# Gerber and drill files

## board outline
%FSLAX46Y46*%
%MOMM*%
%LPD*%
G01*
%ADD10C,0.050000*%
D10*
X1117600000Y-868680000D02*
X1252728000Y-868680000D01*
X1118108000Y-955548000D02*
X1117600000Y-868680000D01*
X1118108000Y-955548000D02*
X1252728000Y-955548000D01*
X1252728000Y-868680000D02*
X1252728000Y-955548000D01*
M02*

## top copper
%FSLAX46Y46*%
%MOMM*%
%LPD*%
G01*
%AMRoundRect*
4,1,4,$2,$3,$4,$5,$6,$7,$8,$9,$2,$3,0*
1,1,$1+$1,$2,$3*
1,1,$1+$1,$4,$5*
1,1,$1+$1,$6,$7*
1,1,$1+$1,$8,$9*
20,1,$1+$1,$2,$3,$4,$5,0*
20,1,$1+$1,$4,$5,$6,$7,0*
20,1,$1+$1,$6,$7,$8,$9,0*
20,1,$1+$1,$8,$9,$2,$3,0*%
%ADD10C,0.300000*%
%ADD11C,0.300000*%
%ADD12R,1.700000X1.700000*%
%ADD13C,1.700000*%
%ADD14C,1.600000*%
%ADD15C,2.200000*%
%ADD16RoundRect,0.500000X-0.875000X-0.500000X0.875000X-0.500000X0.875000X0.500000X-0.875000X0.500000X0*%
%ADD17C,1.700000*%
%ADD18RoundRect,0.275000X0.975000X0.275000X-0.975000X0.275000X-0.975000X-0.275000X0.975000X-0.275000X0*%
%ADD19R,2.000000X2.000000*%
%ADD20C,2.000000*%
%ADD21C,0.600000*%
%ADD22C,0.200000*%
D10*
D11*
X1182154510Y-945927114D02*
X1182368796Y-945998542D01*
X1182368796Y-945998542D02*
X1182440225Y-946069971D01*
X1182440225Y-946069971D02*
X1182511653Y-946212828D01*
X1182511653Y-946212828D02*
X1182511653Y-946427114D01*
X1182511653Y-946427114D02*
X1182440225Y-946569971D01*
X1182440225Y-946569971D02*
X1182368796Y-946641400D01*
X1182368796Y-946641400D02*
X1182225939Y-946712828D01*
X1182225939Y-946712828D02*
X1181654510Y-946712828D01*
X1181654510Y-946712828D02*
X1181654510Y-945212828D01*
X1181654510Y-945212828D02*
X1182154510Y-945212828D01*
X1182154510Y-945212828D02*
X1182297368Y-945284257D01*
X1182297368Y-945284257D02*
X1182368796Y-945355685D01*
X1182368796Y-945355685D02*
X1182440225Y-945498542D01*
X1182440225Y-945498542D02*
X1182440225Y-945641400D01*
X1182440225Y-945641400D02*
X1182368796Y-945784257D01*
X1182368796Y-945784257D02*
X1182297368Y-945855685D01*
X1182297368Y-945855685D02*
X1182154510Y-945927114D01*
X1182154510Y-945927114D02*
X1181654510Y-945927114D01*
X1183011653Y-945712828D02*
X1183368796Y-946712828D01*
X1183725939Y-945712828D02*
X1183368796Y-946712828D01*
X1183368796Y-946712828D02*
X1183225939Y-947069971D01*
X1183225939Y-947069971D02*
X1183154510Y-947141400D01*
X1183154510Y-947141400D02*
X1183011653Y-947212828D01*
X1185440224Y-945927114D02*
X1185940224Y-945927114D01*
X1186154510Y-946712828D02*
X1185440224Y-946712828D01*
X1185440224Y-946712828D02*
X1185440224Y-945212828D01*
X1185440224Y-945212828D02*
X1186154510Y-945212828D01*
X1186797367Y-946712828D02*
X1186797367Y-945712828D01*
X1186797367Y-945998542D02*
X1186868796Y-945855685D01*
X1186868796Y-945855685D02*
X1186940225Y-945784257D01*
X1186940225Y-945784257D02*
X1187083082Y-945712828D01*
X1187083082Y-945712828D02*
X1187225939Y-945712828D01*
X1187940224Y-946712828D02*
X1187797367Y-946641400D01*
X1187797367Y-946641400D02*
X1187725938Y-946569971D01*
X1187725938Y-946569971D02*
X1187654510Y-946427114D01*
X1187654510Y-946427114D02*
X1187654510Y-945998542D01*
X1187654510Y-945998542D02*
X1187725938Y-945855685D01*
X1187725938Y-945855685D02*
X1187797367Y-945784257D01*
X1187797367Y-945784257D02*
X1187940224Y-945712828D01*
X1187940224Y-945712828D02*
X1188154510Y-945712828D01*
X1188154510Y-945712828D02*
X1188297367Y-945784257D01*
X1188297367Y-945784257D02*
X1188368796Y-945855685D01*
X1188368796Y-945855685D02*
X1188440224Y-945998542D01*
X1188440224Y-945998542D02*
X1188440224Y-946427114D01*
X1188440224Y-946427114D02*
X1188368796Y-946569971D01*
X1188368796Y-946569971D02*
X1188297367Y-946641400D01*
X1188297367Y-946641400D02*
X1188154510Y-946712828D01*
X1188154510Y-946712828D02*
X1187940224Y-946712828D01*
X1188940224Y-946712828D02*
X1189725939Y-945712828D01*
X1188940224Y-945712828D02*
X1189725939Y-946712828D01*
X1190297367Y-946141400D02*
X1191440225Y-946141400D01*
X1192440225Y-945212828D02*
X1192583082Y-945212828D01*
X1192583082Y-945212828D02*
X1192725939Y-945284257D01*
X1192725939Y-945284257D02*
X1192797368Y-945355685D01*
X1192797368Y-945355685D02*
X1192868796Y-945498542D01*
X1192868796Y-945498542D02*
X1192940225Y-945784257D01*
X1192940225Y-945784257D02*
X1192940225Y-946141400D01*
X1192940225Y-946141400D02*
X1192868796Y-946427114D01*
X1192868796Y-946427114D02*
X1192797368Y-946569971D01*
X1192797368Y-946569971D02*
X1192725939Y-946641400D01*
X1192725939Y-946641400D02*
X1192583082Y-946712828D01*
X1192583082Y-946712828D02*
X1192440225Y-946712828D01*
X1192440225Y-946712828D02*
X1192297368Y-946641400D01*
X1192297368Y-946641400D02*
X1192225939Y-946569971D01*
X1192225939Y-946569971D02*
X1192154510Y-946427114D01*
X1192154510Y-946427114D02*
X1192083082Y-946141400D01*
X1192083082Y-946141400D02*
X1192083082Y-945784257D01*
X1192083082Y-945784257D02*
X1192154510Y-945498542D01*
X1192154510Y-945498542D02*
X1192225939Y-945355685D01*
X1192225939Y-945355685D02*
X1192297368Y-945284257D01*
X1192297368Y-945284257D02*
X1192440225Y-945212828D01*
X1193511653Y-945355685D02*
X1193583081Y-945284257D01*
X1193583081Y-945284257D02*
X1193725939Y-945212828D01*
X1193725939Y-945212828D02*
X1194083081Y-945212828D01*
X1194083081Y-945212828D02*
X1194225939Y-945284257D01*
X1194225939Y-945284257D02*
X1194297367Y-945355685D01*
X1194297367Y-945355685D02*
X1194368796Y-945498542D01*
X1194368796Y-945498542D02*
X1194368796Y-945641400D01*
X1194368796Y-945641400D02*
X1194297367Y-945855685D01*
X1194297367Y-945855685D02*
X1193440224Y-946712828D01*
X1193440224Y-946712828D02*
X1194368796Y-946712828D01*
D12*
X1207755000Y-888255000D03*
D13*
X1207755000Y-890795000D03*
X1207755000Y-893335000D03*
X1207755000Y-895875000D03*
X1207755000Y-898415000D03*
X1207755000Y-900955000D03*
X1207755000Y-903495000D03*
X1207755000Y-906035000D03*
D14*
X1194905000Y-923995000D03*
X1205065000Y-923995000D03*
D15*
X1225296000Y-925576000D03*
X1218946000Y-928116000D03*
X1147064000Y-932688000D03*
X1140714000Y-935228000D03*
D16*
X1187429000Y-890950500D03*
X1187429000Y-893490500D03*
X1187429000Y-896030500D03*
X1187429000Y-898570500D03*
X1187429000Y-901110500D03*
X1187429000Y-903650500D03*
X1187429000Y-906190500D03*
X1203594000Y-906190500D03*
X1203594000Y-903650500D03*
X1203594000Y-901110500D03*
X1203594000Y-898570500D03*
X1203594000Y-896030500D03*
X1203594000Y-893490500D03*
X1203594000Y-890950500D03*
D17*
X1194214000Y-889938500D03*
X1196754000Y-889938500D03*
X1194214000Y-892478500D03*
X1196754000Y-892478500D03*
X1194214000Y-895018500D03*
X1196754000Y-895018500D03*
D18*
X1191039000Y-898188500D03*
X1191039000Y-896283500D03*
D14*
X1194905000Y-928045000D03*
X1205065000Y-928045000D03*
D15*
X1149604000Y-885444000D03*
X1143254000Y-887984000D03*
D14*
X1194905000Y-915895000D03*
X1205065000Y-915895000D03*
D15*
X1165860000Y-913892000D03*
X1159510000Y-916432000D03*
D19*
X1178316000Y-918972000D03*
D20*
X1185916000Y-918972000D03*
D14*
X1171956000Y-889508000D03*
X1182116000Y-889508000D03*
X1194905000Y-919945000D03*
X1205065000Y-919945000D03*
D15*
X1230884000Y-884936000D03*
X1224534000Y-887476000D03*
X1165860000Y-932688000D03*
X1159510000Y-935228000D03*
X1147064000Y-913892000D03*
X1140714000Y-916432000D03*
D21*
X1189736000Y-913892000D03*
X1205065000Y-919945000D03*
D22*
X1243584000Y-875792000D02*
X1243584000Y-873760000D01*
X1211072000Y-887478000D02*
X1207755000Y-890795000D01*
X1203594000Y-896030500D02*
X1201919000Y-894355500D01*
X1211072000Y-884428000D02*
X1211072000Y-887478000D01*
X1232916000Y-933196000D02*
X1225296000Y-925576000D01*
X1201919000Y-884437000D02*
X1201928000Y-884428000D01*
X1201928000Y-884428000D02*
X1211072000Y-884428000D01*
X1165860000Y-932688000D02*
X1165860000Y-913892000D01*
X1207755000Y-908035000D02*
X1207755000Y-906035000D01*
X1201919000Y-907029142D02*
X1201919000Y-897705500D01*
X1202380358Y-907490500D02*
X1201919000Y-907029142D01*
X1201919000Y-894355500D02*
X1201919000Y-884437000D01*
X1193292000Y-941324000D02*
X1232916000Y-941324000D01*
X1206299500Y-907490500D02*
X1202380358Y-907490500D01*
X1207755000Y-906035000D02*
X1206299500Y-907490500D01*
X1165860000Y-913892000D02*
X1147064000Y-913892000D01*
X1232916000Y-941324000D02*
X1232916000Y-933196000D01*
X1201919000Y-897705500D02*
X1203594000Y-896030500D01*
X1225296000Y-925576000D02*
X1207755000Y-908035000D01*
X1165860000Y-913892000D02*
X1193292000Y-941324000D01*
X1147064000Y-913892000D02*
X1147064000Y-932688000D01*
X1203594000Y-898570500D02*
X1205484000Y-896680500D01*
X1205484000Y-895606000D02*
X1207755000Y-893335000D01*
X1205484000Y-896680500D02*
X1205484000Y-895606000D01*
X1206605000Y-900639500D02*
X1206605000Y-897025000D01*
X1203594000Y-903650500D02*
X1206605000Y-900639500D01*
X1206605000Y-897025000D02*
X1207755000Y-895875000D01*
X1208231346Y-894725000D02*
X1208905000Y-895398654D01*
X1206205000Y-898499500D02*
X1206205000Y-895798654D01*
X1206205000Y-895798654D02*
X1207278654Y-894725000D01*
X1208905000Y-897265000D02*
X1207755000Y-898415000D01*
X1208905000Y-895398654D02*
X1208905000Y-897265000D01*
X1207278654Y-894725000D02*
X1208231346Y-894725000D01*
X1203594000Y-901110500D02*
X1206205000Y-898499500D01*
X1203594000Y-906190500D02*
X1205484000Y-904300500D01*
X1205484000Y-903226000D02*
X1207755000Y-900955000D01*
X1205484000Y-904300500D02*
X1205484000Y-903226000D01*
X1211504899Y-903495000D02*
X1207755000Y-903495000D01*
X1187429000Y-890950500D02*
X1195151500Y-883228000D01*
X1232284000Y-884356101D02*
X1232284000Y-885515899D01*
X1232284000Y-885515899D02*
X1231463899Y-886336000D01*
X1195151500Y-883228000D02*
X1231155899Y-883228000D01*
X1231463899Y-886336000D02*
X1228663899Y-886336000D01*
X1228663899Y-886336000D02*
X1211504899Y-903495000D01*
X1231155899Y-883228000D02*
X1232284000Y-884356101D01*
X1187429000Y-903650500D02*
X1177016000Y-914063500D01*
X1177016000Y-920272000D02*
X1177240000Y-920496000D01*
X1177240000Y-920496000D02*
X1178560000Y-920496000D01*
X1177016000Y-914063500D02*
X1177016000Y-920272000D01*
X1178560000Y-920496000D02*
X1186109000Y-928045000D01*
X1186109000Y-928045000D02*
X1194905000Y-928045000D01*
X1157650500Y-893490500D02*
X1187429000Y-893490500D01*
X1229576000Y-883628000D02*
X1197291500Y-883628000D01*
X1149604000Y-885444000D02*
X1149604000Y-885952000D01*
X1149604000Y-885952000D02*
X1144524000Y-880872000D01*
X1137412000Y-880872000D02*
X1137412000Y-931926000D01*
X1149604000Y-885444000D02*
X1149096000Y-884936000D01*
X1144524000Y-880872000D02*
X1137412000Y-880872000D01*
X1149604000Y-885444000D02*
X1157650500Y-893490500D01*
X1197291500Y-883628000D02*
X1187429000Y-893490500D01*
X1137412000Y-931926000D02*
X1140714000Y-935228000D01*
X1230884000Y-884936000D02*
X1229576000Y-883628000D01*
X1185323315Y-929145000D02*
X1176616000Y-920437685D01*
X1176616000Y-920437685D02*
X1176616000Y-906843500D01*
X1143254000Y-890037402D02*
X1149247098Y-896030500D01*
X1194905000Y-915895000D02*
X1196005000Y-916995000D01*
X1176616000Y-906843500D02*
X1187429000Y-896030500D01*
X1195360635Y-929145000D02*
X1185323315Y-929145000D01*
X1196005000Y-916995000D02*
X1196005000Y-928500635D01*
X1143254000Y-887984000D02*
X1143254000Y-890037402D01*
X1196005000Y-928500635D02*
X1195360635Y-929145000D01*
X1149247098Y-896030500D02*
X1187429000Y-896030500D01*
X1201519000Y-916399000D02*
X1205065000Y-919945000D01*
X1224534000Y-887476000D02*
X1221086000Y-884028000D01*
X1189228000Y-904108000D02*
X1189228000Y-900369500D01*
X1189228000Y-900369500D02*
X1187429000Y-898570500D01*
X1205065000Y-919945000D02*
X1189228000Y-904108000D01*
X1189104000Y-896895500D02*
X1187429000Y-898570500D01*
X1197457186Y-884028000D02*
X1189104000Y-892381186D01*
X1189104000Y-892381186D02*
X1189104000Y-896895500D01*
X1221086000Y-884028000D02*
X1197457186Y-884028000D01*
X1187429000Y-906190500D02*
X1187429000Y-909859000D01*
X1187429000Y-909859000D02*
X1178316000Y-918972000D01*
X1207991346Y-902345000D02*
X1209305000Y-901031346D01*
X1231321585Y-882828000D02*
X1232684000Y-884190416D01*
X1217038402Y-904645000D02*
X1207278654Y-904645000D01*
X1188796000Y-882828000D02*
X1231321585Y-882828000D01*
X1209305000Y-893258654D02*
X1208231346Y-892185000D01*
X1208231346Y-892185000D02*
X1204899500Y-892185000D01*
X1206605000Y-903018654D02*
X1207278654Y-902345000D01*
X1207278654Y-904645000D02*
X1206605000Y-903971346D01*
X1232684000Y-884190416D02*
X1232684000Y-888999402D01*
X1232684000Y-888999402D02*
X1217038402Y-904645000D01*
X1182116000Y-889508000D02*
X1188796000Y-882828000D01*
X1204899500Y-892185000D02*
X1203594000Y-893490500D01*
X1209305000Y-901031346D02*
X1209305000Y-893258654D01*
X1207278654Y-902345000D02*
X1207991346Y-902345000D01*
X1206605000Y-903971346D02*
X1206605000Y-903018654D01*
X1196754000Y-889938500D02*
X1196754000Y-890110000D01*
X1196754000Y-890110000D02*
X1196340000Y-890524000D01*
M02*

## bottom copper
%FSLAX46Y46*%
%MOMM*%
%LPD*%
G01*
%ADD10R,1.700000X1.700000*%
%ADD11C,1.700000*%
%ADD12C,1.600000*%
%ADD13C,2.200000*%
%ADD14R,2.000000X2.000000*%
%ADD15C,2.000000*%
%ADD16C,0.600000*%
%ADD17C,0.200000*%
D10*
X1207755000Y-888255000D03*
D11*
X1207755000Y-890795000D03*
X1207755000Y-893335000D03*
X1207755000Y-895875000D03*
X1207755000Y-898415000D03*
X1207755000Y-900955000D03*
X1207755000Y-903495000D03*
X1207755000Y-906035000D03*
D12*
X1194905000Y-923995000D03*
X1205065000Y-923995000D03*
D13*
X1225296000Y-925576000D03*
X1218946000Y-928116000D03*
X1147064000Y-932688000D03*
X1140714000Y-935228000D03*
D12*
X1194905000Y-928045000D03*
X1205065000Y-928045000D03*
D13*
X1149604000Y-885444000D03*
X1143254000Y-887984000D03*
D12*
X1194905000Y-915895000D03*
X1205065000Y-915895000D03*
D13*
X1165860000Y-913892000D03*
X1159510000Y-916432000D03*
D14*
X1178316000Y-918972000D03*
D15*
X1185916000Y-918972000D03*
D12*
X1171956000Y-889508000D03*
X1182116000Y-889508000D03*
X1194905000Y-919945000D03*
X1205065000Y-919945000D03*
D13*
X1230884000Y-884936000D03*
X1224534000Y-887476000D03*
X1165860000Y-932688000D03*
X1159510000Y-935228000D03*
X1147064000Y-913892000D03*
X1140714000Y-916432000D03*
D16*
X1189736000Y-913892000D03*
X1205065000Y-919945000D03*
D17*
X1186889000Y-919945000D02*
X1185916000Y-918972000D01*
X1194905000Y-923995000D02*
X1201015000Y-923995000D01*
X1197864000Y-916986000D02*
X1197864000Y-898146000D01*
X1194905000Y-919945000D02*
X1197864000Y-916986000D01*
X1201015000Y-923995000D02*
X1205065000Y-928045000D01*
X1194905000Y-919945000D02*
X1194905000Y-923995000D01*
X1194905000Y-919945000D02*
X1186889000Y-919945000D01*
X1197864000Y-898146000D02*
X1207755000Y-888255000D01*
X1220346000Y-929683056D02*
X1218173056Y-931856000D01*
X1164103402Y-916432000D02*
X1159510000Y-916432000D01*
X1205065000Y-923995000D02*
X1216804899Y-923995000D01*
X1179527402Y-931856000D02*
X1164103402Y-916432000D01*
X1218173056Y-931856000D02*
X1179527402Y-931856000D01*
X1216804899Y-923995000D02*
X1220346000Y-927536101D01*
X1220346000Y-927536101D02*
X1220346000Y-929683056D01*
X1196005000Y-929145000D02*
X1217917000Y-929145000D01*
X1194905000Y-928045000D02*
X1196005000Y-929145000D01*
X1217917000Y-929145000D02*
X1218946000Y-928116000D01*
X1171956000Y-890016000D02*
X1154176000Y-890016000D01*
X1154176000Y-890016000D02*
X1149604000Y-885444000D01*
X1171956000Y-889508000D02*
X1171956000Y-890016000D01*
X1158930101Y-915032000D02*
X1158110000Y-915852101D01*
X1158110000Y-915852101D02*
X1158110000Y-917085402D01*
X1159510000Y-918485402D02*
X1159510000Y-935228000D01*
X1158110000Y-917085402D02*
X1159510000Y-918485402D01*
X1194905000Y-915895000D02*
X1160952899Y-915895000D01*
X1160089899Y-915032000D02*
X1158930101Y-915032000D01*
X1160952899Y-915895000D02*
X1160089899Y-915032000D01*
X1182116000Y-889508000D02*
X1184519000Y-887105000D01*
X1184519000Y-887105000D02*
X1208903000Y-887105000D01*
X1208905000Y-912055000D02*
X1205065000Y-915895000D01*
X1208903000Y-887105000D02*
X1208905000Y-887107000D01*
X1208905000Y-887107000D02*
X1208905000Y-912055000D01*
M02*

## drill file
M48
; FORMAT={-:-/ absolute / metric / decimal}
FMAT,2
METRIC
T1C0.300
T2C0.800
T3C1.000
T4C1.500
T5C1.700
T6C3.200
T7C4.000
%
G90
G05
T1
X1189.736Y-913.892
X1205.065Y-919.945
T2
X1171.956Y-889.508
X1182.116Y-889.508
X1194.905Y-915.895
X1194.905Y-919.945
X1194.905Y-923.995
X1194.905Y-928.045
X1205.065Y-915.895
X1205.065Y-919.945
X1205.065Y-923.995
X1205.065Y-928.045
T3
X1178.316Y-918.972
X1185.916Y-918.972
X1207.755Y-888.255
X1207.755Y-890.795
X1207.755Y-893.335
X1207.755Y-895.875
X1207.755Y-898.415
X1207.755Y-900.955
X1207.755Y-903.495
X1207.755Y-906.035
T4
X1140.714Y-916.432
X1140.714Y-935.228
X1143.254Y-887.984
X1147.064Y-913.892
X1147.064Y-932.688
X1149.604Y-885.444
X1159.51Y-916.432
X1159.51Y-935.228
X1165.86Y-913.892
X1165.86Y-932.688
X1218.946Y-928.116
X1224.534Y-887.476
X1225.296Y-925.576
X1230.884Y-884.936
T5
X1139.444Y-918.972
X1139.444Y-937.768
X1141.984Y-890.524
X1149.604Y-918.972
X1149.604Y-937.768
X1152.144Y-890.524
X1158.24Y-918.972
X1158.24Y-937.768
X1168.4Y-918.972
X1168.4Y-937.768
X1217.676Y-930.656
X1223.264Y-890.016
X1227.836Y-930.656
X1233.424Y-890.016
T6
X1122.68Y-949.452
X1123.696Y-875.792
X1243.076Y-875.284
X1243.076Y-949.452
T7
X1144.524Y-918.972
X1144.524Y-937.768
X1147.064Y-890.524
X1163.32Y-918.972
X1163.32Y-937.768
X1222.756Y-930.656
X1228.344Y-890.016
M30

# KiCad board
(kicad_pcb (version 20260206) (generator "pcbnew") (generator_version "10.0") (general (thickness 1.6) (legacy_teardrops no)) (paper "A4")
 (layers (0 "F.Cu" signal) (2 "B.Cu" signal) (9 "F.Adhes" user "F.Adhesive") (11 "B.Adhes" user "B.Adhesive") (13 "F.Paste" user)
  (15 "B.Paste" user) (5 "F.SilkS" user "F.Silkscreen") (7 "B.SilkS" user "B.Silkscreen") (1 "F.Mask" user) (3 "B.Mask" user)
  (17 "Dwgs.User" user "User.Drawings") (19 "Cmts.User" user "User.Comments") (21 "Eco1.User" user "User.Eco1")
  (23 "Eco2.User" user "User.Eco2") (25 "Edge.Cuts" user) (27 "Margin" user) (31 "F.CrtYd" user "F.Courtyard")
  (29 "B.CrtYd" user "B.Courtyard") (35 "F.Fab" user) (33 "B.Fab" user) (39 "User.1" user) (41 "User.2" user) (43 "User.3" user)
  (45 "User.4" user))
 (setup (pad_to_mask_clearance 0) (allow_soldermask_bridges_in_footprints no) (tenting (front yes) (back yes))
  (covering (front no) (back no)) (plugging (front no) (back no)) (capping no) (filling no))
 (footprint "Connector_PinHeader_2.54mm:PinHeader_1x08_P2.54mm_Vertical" (layer "F.Cu") (at 1207.755 888.255)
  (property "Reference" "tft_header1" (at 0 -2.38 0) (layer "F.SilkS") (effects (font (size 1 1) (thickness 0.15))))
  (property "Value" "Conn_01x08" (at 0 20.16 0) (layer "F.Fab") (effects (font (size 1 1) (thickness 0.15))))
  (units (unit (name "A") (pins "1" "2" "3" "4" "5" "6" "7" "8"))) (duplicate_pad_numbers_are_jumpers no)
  (pad "1" thru_hole rect (at 0 0) (size 1.7 1.7) (drill 1) (layers "*.Cu" "*.Mask") (remove_unused_layers no) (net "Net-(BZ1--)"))
  (pad "2" thru_hole circle (at 0 2.54) (size 1.7 1.7) (drill 1) (layers "*.Cu" "*.Mask") (remove_unused_layers no) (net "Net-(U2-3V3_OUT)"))
  (pad "3" thru_hole circle (at 0 5.08) (size 1.7 1.7) (drill 1) (layers "*.Cu" "*.Mask") (remove_unused_layers no) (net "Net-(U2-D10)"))
  (pad "4" thru_hole circle (at 0 7.62) (size 1.7 1.7) (drill 1) (layers "*.Cu" "*.Mask") (remove_unused_layers no) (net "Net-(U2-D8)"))
  (pad "5" thru_hole circle (at 0 10.16) (size 1.7 1.7) (drill 1) (layers "*.Cu" "*.Mask") (remove_unused_layers no)
   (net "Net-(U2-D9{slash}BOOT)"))
  (pad "6" thru_hole circle (at 0 12.7) (size 1.7 1.7) (drill 1) (layers "*.Cu" "*.Mask") (remove_unused_layers no) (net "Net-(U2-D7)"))
  (pad "7" thru_hole circle (at 0 15.24) (size 1.7 1.7) (drill 1) (layers "*.Cu" "*.Mask") (remove_unused_layers no) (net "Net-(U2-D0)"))
  (pad "8" thru_hole circle (at 0 17.78) (size 1.7 1.7) (drill 1) (layers "*.Cu" "*.Mask") (remove_unused_layers no)
   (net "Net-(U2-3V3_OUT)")))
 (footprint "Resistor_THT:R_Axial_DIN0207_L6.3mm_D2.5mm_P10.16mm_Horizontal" (layer "F.Cu") (at 1194.905 923.995)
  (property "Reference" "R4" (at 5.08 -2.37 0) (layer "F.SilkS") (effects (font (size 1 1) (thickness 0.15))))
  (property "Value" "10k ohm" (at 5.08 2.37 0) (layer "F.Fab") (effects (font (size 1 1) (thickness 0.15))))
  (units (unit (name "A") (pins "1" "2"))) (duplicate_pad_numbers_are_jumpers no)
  (pad "1" thru_hole circle (at 0 0) (size 1.6 1.6) (drill 0.8) (layers "*.Cu" "*.Mask") (remove_unused_layers no) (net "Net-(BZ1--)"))
  (pad "2" thru_hole circle (at 10.16 0) (size 1.6 1.6) (drill 0.8) (layers "*.Cu" "*.Mask") (remove_unused_layers no) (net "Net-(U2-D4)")))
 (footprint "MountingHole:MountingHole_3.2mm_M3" (layer "F.Cu") (at 1122.68 949.452)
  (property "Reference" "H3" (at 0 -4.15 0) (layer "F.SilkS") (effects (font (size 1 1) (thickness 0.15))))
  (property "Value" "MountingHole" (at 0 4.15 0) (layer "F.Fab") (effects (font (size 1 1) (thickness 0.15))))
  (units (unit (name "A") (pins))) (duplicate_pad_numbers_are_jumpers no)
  (pad "" np_thru_hole circle (at 0 0) (size 3.2 3.2) (drill 3.2) (layers "*.Cu" "*.Mask")))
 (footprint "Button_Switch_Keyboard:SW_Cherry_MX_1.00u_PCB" (layer "F.Cu") (at 1225.296 925.576)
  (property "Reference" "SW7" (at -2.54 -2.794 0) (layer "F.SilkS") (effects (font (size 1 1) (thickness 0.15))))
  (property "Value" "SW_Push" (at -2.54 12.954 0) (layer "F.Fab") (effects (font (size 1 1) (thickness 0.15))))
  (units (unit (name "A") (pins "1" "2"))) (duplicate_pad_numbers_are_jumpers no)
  (pad "" np_thru_hole circle (at -7.62 5.08) (size 1.7 1.7) (drill 1.7) (layers "*.Cu" "*.Mask"))
  (pad "" np_thru_hole circle (at -2.54 5.08) (size 4 4) (drill 4) (layers "*.Cu" "*.Mask"))
  (pad "" np_thru_hole circle (at 2.54 5.08) (size 1.7 1.7) (drill 1.7) (layers "*.Cu" "*.Mask"))
  (pad "1" thru_hole circle (at 0 0) (size 2.2 2.2) (drill 1.5) (layers "*.Cu" "*.Mask") (remove_unused_layers no) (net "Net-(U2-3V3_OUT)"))
  (pad "2" thru_hole circle (at -6.35 2.54) (size 2.2 2.2) (drill 1.5) (layers "*.Cu" "*.Mask") (remove_unused_layers no)
   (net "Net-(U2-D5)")))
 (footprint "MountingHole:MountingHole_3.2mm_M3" (layer "F.Cu") (at 1123.696 875.792)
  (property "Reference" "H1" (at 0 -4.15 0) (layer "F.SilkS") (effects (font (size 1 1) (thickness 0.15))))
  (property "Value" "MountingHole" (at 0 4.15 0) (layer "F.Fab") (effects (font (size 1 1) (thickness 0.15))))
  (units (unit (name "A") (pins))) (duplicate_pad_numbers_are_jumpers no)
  (pad "" np_thru_hole circle (at 0 0) (size 3.2 3.2) (drill 3.2) (layers "*.Cu" "*.Mask")))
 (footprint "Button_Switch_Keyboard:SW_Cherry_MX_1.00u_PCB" (layer "F.Cu") (at 1147.064 932.688)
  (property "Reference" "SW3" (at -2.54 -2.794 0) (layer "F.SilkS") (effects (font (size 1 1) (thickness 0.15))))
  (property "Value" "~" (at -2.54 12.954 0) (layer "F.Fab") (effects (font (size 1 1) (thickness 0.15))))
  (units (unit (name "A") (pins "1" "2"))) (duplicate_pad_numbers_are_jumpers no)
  (pad "" np_thru_hole circle (at -7.62 5.08) (size 1.7 1.7) (drill 1.7) (layers "*.Cu" "*.Mask"))
  (pad "" np_thru_hole circle (at -2.54 5.08) (size 4 4) (drill 4) (layers "*.Cu" "*.Mask"))
  (pad "" np_thru_hole circle (at 2.54 5.08) (size 1.7 1.7) (drill 1.7) (layers "*.Cu" "*.Mask"))
  (pad "1" thru_hole circle (at 0 0) (size 2.2 2.2) (drill 1.5) (layers "*.Cu" "*.Mask") (remove_unused_layers no) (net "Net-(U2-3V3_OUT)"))
  (pad "2" thru_hole circle (at -6.35 2.54) (size 2.2 2.2) (drill 1.5) (layers "*.Cu" "*.Mask") (remove_unused_layers no)
   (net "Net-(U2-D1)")))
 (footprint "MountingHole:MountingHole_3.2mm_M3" (layer "F.Cu") (at 1243.076 875.284)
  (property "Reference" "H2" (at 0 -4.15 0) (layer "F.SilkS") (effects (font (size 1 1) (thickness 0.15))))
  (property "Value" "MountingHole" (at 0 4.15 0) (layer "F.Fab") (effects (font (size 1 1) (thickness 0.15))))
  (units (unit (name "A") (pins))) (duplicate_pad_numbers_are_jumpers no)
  (pad "" np_thru_hole circle (at 0 0) (size 3.2 3.2) (drill 3.2) (layers "*.Cu" "*.Mask")))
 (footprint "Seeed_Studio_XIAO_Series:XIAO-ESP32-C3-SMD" (layer "F.Cu") (at 1186.594 909.0705)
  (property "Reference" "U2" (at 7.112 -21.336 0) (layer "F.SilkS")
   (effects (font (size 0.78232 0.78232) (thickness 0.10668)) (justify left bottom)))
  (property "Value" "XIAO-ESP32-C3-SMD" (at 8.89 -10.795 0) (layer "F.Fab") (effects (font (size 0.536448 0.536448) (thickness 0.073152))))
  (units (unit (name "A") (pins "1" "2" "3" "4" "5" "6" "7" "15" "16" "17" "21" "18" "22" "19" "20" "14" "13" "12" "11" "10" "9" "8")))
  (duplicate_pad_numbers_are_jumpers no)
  (pad "1" smd roundrect (at 0.835 -18.12) (size 2.75 2) (layers "F.Cu" "F.Mask" "F.Paste") (roundrect_rratio 0.25) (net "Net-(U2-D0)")
   (solder_mask_margin 0.0508) (thermal_bridge_angle 45))
  (pad "2" smd roundrect (at 0.835 -15.58) (size 2.75 2) (layers "F.Cu" "F.Mask" "F.Paste") (roundrect_rratio 0.25) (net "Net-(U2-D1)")
   (solder_mask_margin 0.0508) (thermal_bridge_angle 45))
  (pad "3" smd roundrect (at 0.835 -13.04) (size 2.75 2) (layers "F.Cu" "F.Mask" "F.Paste") (roundrect_rratio 0.25) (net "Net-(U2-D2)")
   (solder_mask_margin 0.0508) (thermal_bridge_angle 45))
  (pad "4" smd roundrect (at 0.835 -10.5) (size 2.75 2) (layers "F.Cu" "F.Mask" "F.Paste") (roundrect_rratio 0.25) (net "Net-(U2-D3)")
   (solder_mask_margin 0.0508) (thermal_bridge_angle 45))
  (pad "5" smd roundrect (at 0.835 -7.96) (size 2.75 2) (layers "F.Cu" "F.Mask" "F.Paste") (roundrect_rratio 0.25) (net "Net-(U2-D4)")
   (solder_mask_margin 0.0508) (thermal_bridge_angle 45))
  (pad "6" smd roundrect (at 0.835 -5.42) (size 2.75 2) (layers "F.Cu" "F.Mask" "F.Paste") (roundrect_rratio 0.25) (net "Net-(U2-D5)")
   (solder_mask_margin 0.0508) (thermal_bridge_angle 45))
  (pad "7" smd roundrect (at 0.835 -2.88) (size 2.75 2) (layers "F.Cu" "F.Mask" "F.Paste") (roundrect_rratio 0.25) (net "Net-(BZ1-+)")
   (solder_mask_margin 0.0508) (thermal_bridge_angle 45))
  (pad "8" smd roundrect (at 17 -2.88) (size 2.75 2) (layers "F.Cu" "F.Mask" "F.Paste") (roundrect_rratio 0.25) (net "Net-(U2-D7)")
   (solder_mask_margin 0.0508) (thermal_bridge_angle 45))
  (pad "9" smd roundrect (at 17 -5.42) (size 2.75 2) (layers "F.Cu" "F.Mask" "F.Paste") (roundrect_rratio 0.25) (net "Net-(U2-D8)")
   (solder_mask_margin 0.0508) (thermal_bridge_angle 45))
  (pad "10" smd roundrect (at 17 -7.96) (size 2.75 2) (layers "F.Cu" "F.Mask" "F.Paste") (roundrect_rratio 0.25)
   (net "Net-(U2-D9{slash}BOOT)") (solder_mask_margin 0.0508) (thermal_bridge_angle 45))
  (pad "11" smd roundrect (at 17 -10.5) (size 2.75 2) (layers "F.Cu" "F.Mask" "F.Paste") (roundrect_rratio 0.25) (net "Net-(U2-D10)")
   (solder_mask_margin 0.0508) (thermal_bridge_angle 45))
  (pad "12" smd roundrect (at 17 -13.04) (size 2.75 2) (layers "F.Cu" "F.Mask" "F.Paste") (roundrect_rratio 0.25) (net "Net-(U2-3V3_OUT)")
   (solder_mask_margin 0.0508) (thermal_bridge_angle 45))
  (pad "13" smd roundrect (at 17 -15.58) (size 2.75 2) (layers "F.Cu" "F.Mask" "F.Paste") (roundrect_rratio 0.25) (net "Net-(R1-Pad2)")
   (solder_mask_margin 0.0508) (thermal_bridge_angle 45))
  (pad "14" smd roundrect (at 17 -18.12) (size 2.75 2) (layers "F.Cu" "F.Mask" "F.Paste") (roundrect_rratio 0.25)
   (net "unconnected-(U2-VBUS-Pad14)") (solder_mask_margin 0.0508) (thermal_bridge_angle 45))
  (pad "15" smd circle (at 7.62 -19.132) (size 1.7 1.7) (layers "F.Cu" "F.Mask" "F.Paste") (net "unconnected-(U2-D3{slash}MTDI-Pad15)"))
  (pad "16" smd circle (at 10.16 -19.132) (size 1.7 1.7) (layers "F.Cu" "F.Mask" "F.Paste") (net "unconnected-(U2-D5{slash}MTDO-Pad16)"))
  (pad "17" smd circle (at 7.62 -16.592) (size 1.7 1.7) (layers "F.Cu" "F.Mask" "F.Paste") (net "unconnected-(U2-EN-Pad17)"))
  (pad "18" smd circle (at 10.16 -16.592) (size 1.7 1.7) (layers "F.Cu" "F.Mask" "F.Paste") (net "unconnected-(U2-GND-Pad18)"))
  (pad "19" smd circle (at 7.62 -14.052) (size 1.7 1.7) (layers "F.Cu" "F.Mask" "F.Paste") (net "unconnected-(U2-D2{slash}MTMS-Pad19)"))
  (pad "20" smd circle (at 10.16 -14.052) (size 1.7 1.7) (layers "F.Cu" "F.Mask" "F.Paste") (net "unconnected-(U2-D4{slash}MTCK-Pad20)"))
  (pad "21" smd roundrect (at 4.445 -10.882 180) (size 2.5 1.1) (layers "F.Cu" "F.Mask" "F.Paste") (roundrect_rratio 0.25) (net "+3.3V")
   (thermal_bridge_angle 45))
  (pad "22" smd roundrect (at 4.445 -12.787 180) (size 2.5 1.1) (layers "F.Cu" "F.Mask" "F.Paste") (roundrect_rratio 0.25) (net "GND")
   (thermal_bridge_angle 45)))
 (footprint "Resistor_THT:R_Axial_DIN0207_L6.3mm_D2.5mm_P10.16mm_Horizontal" (layer "F.Cu") (at 1194.905 928.045)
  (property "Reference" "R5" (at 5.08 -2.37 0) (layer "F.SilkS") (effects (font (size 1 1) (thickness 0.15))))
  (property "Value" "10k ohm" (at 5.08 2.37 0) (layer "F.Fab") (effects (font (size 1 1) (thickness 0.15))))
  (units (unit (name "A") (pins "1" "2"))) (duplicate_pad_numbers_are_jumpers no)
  (pad "1" thru_hole circle (at 0 0) (size 1.6 1.6) (drill 0.8) (layers "*.Cu" "*.Mask") (remove_unused_layers no) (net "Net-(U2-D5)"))
  (pad "2" thru_hole circle (at 10.16 0) (size 1.6 1.6) (drill 0.8) (layers "*.Cu" "*.Mask") (remove_unused_layers no) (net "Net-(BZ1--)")))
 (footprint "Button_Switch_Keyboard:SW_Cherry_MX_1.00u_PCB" (layer "F.Cu") (at 1149.604 885.444)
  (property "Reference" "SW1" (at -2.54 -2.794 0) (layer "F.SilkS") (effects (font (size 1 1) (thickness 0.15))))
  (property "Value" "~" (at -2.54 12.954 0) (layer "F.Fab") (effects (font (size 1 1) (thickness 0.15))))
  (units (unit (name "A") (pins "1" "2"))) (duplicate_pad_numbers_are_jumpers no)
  (pad "" np_thru_hole circle (at -7.62 5.08) (size 1.7 1.7) (drill 1.7) (layers "*.Cu" "*.Mask"))
  (pad "" np_thru_hole circle (at -2.54 5.08) (size 4 4) (drill 4) (layers "*.Cu" "*.Mask"))
  (pad "" np_thru_hole circle (at 2.54 5.08) (size 1.7 1.7) (drill 1.7) (layers "*.Cu" "*.Mask"))
  (pad "1" thru_hole circle (at 0 0) (size 2.2 2.2) (drill 1.5) (layers "*.Cu" "*.Mask") (remove_unused_layers no) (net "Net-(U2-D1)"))
  (pad "2" thru_hole circle (at -6.35 2.54) (size 2.2 2.2) (drill 1.5) (layers "*.Cu" "*.Mask") (remove_unused_layers no)
   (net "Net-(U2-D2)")))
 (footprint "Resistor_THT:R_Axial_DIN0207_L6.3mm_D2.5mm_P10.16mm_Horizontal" (layer "F.Cu") (at 1194.905 915.895)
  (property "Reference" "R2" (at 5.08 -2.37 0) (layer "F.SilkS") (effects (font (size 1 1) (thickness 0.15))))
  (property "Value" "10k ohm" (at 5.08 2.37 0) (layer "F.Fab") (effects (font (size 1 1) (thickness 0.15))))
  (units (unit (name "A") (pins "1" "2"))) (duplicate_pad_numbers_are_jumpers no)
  (pad "1" thru_hole circle (at 0 0) (size 1.6 1.6) (drill 0.8) (layers "*.Cu" "*.Mask") (remove_unused_layers no) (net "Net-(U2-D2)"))
  (pad "2" thru_hole circle (at 10.16 0) (size 1.6 1.6) (drill 0.8) (layers "*.Cu" "*.Mask") (remove_unused_layers no) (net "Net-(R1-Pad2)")))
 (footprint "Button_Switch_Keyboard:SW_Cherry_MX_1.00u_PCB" (layer "F.Cu") (at 1165.86 913.892)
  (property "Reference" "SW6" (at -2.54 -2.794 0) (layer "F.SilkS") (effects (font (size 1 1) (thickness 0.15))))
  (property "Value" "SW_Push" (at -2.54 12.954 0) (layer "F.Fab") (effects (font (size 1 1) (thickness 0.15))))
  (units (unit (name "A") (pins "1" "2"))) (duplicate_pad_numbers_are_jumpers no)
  (pad "" np_thru_hole circle (at -7.62 5.08) (size 1.7 1.7) (drill 1.7) (layers "*.Cu" "*.Mask"))
  (pad "" np_thru_hole circle (at -2.54 5.08) (size 4 4) (drill 4) (layers "*.Cu" "*.Mask"))
  (pad "" np_thru_hole circle (at 2.54 5.08) (size 1.7 1.7) (drill 1.7) (layers "*.Cu" "*.Mask"))
  (pad "1" thru_hole circle (at 0 0) (size 2.2 2.2) (drill 1.5) (layers "*.Cu" "*.Mask") (remove_unused_layers no) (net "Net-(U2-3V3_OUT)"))
  (pad "2" thru_hole circle (at -6.35 2.54) (size 2.2 2.2) (drill 1.5) (layers "*.Cu" "*.Mask") (remove_unused_layers no)
   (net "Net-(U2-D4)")))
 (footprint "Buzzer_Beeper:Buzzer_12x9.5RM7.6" (layer "F.Cu") (at 1178.316 918.972)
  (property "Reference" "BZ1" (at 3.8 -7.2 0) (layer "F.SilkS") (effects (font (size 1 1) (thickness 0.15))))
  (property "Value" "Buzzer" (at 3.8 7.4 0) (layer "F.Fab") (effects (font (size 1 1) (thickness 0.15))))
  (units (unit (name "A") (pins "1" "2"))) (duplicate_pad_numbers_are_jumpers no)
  (pad "1" thru_hole rect (at 0 0) (size 2 2) (drill 1) (layers "*.Cu" "*.Mask") (remove_unused_layers no) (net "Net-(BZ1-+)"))
  (pad "2" thru_hole circle (at 7.6 0) (size 2 2) (drill 1) (layers "*.Cu" "*.Mask") (remove_unused_layers no) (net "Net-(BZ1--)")))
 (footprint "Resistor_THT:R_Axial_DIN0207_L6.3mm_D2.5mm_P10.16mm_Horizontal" (layer "F.Cu") (at 1171.956 889.508)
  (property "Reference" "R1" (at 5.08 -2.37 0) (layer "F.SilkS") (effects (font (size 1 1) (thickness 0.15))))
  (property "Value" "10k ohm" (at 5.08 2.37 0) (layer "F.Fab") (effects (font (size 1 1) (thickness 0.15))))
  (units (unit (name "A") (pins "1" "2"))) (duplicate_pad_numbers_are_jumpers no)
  (pad "1" thru_hole circle (at 0 0) (size 1.6 1.6) (drill 0.8) (layers "*.Cu" "*.Mask") (remove_unused_layers no) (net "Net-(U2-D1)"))
  (pad "2" thru_hole circle (at 10.16 0) (size 1.6 1.6) (drill 0.8) (layers "*.Cu" "*.Mask") (remove_unused_layers no) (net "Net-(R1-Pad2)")))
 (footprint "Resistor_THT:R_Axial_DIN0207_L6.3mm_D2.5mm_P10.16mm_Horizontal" (layer "F.Cu") (at 1194.905 919.945)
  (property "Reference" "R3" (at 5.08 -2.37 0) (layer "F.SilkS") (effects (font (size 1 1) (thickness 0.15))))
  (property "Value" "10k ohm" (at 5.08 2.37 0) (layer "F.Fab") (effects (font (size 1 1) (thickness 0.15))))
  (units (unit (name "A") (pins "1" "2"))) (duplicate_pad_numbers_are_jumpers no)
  (pad "1" thru_hole circle (at 0 0) (size 1.6 1.6) (drill 0.8) (layers "*.Cu" "*.Mask") (remove_unused_layers no) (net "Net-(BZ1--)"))
  (pad "2" thru_hole circle (at 10.16 0) (size 1.6 1.6) (drill 0.8) (layers "*.Cu" "*.Mask") (remove_unused_layers no) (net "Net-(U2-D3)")))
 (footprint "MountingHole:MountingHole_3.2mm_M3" (layer "F.Cu") (at 1243.076 949.452)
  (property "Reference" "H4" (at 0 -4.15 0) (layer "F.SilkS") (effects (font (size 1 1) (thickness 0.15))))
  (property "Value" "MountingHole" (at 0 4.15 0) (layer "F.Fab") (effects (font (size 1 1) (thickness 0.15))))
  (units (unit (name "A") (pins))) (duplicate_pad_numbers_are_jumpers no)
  (pad "" np_thru_hole circle (at 0 0) (size 3.2 3.2) (drill 3.2) (layers "*.Cu" "*.Mask")))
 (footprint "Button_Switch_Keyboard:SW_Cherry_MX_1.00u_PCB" (layer "F.Cu") (at 1230.884 884.936)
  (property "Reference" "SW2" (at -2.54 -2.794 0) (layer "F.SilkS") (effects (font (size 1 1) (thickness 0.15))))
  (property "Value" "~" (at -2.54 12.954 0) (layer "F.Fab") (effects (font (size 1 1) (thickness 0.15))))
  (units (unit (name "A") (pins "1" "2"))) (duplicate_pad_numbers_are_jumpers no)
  (pad "" np_thru_hole circle (at -7.62 5.08) (size 1.7 1.7) (drill 1.7) (layers "*.Cu" "*.Mask"))
  (pad "" np_thru_hole circle (at -2.54 5.08) (size 4 4) (drill 4) (layers "*.Cu" "*.Mask"))
  (pad "" np_thru_hole circle (at 2.54 5.08) (size 1.7 1.7) (drill 1.7) (layers "*.Cu" "*.Mask"))
  (pad "1" thru_hole circle (at 0 0) (size 2.2 2.2) (drill 1.5) (layers "*.Cu" "*.Mask") (remove_unused_layers no) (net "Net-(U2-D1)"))
  (pad "2" thru_hole circle (at -6.35 2.54) (size 2.2 2.2) (drill 1.5) (layers "*.Cu" "*.Mask") (remove_unused_layers no)
   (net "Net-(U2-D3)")))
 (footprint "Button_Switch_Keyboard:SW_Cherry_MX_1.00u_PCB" (layer "F.Cu") (at 1165.86 932.688)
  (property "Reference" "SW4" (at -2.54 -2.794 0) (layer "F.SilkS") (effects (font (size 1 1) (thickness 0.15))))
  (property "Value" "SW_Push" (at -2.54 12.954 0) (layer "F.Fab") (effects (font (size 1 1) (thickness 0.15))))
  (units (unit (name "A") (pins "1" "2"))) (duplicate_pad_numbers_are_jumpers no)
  (pad "" np_thru_hole circle (at -7.62 5.08) (size 1.7 1.7) (drill 1.7) (layers "*.Cu" "*.Mask"))
  (pad "" np_thru_hole circle (at -2.54 5.08) (size 4 4) (drill 4) (layers "*.Cu" "*.Mask"))
  (pad "" np_thru_hole circle (at 2.54 5.08) (size 1.7 1.7) (drill 1.7) (layers "*.Cu" "*.Mask"))
  (pad "1" thru_hole circle (at 0 0) (size 2.2 2.2) (drill 1.5) (layers "*.Cu" "*.Mask") (remove_unused_layers no) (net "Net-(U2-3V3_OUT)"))
  (pad "2" thru_hole circle (at -6.35 2.54) (size 2.2 2.2) (drill 1.5) (layers "*.Cu" "*.Mask") (remove_unused_layers no)
   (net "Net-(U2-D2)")))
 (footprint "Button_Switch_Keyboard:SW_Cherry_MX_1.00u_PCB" (layer "F.Cu") (at 1147.064 913.892)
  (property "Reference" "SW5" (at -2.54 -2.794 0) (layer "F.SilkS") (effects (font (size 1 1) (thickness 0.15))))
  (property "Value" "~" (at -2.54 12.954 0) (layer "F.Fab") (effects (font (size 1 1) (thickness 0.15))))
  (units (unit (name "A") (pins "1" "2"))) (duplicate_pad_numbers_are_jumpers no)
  (pad "" np_thru_hole circle (at -7.62 5.08) (size 1.7 1.7) (drill 1.7) (layers "*.Cu" "*.Mask"))
  (pad "" np_thru_hole circle (at -2.54 5.08) (size 4 4) (drill 4) (layers "*.Cu" "*.Mask"))
  (pad "" np_thru_hole circle (at 2.54 5.08) (size 1.7 1.7) (drill 1.7) (layers "*.Cu" "*.Mask"))
  (pad "1" thru_hole circle (at 0 0) (size 2.2 2.2) (drill 1.5) (layers "*.Cu" "*.Mask") (remove_unused_layers no) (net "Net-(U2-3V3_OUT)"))
  (pad "2" thru_hole circle (at -6.35 2.54) (size 2.2 2.2) (drill 1.5) (layers "*.Cu" "*.Mask") (remove_unused_layers no)
   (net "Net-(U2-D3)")))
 (gr_line (start 1117.6 868.68) (end 1252.728 868.68) (stroke (width 0.05) (type default)) (layer "Edge.Cuts"))
 (gr_line (start 1118.108 955.548) (end 1117.6 868.68) (stroke (width 0.05) (type default)) (layer "Edge.Cuts"))
 (gr_line (start 1118.108 955.548) (end 1252.728 955.548) (stroke (width 0.05) (type default)) (layer "Edge.Cuts"))
 (gr_line (start 1252.728 868.68) (end 1252.728 955.548) (stroke (width 0.05) (type default)) (layer "Edge.Cuts"))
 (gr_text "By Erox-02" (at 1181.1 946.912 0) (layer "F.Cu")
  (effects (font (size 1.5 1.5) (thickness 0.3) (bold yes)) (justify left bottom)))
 (segment (start 1243.584 875.792) (end 1243.584 873.76) (width 0.2) (layer "F.Cu") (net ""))
 (via (at 1189.736 913.892) (size 0.6) (drill 0.3) (layers "F.Cu" "B.Cu") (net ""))
 (segment (start 1186.889 919.945) (end 1185.916 918.972) (width 0.2) (layer "B.Cu") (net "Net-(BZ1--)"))
 (segment (start 1194.905 923.995) (end 1201.015 923.995) (width 0.2) (layer "B.Cu") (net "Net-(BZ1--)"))
 (segment (start 1197.864 916.986) (end 1197.864 898.146) (width 0.2) (layer "B.Cu") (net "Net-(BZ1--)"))
 (segment (start 1194.905 919.945) (end 1197.864 916.986) (width 0.2) (layer "B.Cu") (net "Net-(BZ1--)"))
 (segment (start 1201.015 923.995) (end 1205.065 928.045) (width 0.2) (layer "B.Cu") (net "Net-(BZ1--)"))
 (segment (start 1194.905 919.945) (end 1194.905 923.995) (width 0.2) (layer "B.Cu") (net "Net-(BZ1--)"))
 (segment (start 1194.905 919.945) (end 1186.889 919.945) (width 0.2) (layer "B.Cu") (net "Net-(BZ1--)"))
 (segment (start 1197.864 898.146) (end 1207.755 888.255) (width 0.2) (layer "B.Cu") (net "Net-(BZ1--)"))
 (segment (start 1211.072 887.478) (end 1207.755 890.795) (width 0.2) (layer "F.Cu") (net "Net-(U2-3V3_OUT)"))
 (segment (start 1203.594 896.0305) (end 1201.919 894.3555) (width 0.2) (layer "F.Cu") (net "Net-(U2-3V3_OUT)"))
 (segment (start 1211.072 884.428) (end 1211.072 887.478) (width 0.2) (layer "F.Cu") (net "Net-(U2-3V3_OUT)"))
 (segment (start 1232.916 933.196) (end 1225.296 925.576) (width 0.2) (layer "F.Cu") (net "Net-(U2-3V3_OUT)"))
 (segment (start 1201.919 884.437) (end 1201.928 884.428) (width 0.2) (layer "F.Cu") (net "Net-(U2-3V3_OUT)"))
 (segment (start 1201.928 884.428) (end 1211.072 884.428) (width 0.2) (layer "F.Cu") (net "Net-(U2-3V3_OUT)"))
 (segment (start 1165.86 932.688) (end 1165.86 913.892) (width 0.2) (layer "F.Cu") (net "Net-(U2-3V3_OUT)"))
 (segment (start 1207.755 908.035) (end 1207.755 906.035) (width 0.2) (layer "F.Cu") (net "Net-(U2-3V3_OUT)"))
 (segment (start 1201.919 907.029142) (end 1201.919 897.7055) (width 0.2) (layer "F.Cu") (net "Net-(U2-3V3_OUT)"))
 (segment (start 1202.380358 907.4905) (end 1201.919 907.029142) (width 0.2) (layer "F.Cu") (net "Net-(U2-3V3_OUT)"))
 (segment (start 1201.919 894.3555) (end 1201.919 884.437) (width 0.2) (layer "F.Cu") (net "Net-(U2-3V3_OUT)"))
 (segment (start 1193.292 941.324) (end 1232.916 941.324) (width 0.2) (layer "F.Cu") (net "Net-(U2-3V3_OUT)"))
 (segment (start 1206.2995 907.4905) (end 1202.380358 907.4905) (width 0.2) (layer "F.Cu") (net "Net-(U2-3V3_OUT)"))
 (segment (start 1207.755 906.035) (end 1206.2995 907.4905) (width 0.2) (layer "F.Cu") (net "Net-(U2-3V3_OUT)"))
 (segment (start 1165.86 913.892) (end 1147.064 913.892) (width 0.2) (layer "F.Cu") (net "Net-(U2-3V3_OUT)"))
 (segment (start 1232.916 941.324) (end 1232.916 933.196) (width 0.2) (layer "F.Cu") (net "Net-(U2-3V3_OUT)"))
 (segment (start 1201.919 897.7055) (end 1203.594 896.0305) (width 0.2) (layer "F.Cu") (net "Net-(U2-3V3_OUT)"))
 (segment (start 1225.296 925.576) (end 1207.755 908.035) (width 0.2) (layer "F.Cu") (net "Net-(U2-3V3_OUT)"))
 (segment (start 1165.86 913.892) (end 1193.292 941.324) (width 0.2) (layer "F.Cu") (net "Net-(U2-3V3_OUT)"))
 (segment (start 1147.064 913.892) (end 1147.064 932.688) (width 0.2) (layer "F.Cu") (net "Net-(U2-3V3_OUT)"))
 (segment (start 1203.594 898.5705) (end 1205.484 896.6805) (width 0.2) (layer "F.Cu") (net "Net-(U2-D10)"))
 (segment (start 1205.484 895.606) (end 1207.755 893.335) (width 0.2) (layer "F.Cu") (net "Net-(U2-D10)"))
 (segment (start 1205.484 896.6805) (end 1205.484 895.606) (width 0.2) (layer "F.Cu") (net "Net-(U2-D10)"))
 (segment (start 1206.605 900.6395) (end 1206.605 897.025) (width 0.2) (layer "F.Cu") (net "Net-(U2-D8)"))
 (segment (start 1203.594 903.6505) (end 1206.605 900.6395) (width 0.2) (layer "F.Cu") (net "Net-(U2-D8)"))
 (segment (start 1206.605 897.025) (end 1207.755 895.875) (width 0.2) (layer "F.Cu") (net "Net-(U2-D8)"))
 (segment (start 1208.231346 894.725) (end 1208.905 895.398654) (width 0.2) (layer "F.Cu") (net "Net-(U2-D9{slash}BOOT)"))
 (segment (start 1206.205 898.4995) (end 1206.205 895.798654) (width 0.2) (layer "F.Cu") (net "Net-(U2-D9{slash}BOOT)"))
 (segment (start 1206.205 895.798654) (end 1207.278654 894.725) (width 0.2) (layer "F.Cu") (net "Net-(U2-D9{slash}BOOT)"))
 (segment (start 1208.905 897.265) (end 1207.755 898.415) (width 0.2) (layer "F.Cu") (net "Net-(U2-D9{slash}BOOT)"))
 (segment (start 1208.905 895.398654) (end 1208.905 897.265) (width 0.2) (layer "F.Cu") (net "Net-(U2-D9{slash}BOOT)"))
 (segment (start 1207.278654 894.725) (end 1208.231346 894.725) (width 0.2) (layer "F.Cu") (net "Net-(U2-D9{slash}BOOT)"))
 (segment (start 1203.594 901.1105) (end 1206.205 898.4995) (width 0.2) (layer "F.Cu") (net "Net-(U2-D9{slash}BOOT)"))
 (segment (start 1203.594 906.1905) (end 1205.484 904.3005) (width 0.2) (layer "F.Cu") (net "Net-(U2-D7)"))
 (segment (start 1205.484 903.226) (end 1207.755 900.955) (width 0.2) (layer "F.Cu") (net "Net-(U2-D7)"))
 (segment (start 1205.484 904.3005) (end 1205.484 903.226) (width 0.2) (layer "F.Cu") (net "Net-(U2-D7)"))
 (segment (start 1211.504899 903.495) (end 1207.755 903.495) (width 0.2) (layer "F.Cu") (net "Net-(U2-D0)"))
 (segment (start 1187.429 890.9505) (end 1195.1515 883.228) (width 0.2) (layer "F.Cu") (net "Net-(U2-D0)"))
 (segment (start 1232.284 884.356101) (end 1232.284 885.515899) (width 0.2) (layer "F.Cu") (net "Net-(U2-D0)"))
 (segment (start 1232.284 885.515899) (end 1231.463899 886.336) (width 0.2) (layer "F.Cu") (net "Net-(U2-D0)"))
 (segment (start 1195.1515 883.228) (end 1231.155899 883.228) (width 0.2) (layer "F.Cu") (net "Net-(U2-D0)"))
 (segment (start 1231.463899 886.336) (end 1228.663899 886.336) (width 0.2) (layer "F.Cu") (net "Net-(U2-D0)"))
 (segment (start 1228.663899 886.336) (end 1211.504899 903.495) (width 0.2) (layer "F.Cu") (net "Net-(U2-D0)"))
 (segment (start 1231.155899 883.228) (end 1232.284 884.356101) (width 0.2) (layer "F.Cu") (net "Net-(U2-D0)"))
 (segment (start 1220.346 929.683056) (end 1218.173056 931.856) (width 0.2) (layer "B.Cu") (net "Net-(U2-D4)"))
 (segment (start 1164.103402 916.432) (end 1159.51 916.432) (width 0.2) (layer "B.Cu") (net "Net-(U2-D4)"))
 (segment (start 1205.065 923.995) (end 1216.804899 923.995) (width 0.2) (layer "B.Cu") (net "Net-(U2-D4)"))
 (segment (start 1179.527402 931.856) (end 1164.103402 916.432) (width 0.2) (layer "B.Cu") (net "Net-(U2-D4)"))
 (segment (start 1218.173056 931.856) (end 1179.527402 931.856) (width 0.2) (layer "B.Cu") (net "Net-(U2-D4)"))
 (segment (start 1216.804899 923.995) (end 1220.346 927.536101) (width 0.2) (layer "B.Cu") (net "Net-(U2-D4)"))
 (segment (start 1220.346 927.536101) (end 1220.346 929.683056) (width 0.2) (layer "B.Cu") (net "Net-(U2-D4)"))
 (segment (start 1187.429 903.6505) (end 1177.016 914.0635) (width 0.2) (layer "F.Cu") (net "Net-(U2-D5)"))
 (segment (start 1177.016 920.272) (end 1177.24 920.496) (width 0.2) (layer "F.Cu") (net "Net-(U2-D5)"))
 (segment (start 1177.24 920.496) (end 1178.56 920.496) (width 0.2) (layer "F.Cu") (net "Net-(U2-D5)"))
 (segment (start 1177.016 914.0635) (end 1177.016 920.272) (width 0.2) (layer "F.Cu") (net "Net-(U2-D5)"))
 (segment (start 1178.56 920.496) (end 1186.109 928.045) (width 0.2) (layer "F.Cu") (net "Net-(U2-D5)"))
 (segment (start 1186.109 928.045) (end 1194.905 928.045) (width 0.2) (layer "F.Cu") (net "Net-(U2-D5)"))
 (segment (start 1196.005 929.145) (end 1217.917 929.145) (width 0.2) (layer "B.Cu") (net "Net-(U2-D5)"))
 (segment (start 1194.905 928.045) (end 1196.005 929.145) (width 0.2) (layer "B.Cu") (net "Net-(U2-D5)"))
 (segment (start 1217.917 929.145) (end 1218.946 928.116) (width 0.2) (layer "B.Cu") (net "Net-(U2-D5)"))
 (segment (start 1157.6505 893.4905) (end 1187.429 893.4905) (width 0.2) (layer "F.Cu") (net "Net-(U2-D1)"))
 (segment (start 1229.576 883.628) (end 1197.2915 883.628) (width 0.2) (layer "F.Cu") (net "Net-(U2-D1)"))
 (segment (start 1149.604 885.444) (end 1149.604 885.952) (width 0.2) (layer "F.Cu") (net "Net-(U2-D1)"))
 (segment (start 1149.604 885.952) (end 1144.524 880.872) (width 0.2) (layer "F.Cu") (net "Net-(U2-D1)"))
 (segment (start 1137.412 880.872) (end 1137.412 931.926) (width 0.2) (layer "F.Cu") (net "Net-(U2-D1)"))
 (segment (start 1149.604 885.444) (end 1149.096 884.936) (width 0.2) (layer "F.Cu") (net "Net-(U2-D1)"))
 (segment (start 1144.524 880.872) (end 1137.412 880.872) (width 0.2) (layer "F.Cu") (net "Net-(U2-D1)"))
 (segment (start 1149.604 885.444) (end 1157.6505 893.4905) (width 0.2) (layer "F.Cu") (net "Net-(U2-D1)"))
 (segment (start 1197.2915 883.628) (end 1187.429 893.4905) (width 0.2) (layer "F.Cu") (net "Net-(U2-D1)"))
 (segment (start 1137.412 931.926) (end 1140.714 935.228) (width 0.2) (layer "F.Cu") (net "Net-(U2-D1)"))
 (segment (start 1230.884 884.936) (end 1229.576 883.628) (width 0.2) (layer "F.Cu") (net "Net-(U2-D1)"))
 (segment (start 1171.956 890.016) (end 1154.176 890.016) (width 0.2) (layer "B.Cu") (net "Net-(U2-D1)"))
 (segment (start 1154.176 890.016) (end 1149.604 885.444) (width 0.2) (layer "B.Cu") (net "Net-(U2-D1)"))
 (segment (start 1171.956 889.508) (end 1171.956 890.016) (width 0.2) (layer "B.Cu") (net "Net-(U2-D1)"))
 (segment (start 1185.323315 929.145) (end 1176.616 920.437685) (width 0.2) (layer "F.Cu") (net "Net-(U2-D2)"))
 (segment (start 1176.616 920.437685) (end 1176.616 906.8435) (width 0.2) (layer "F.Cu") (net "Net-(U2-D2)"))
 (segment (start 1143.254 890.037402) (end 1149.247098 896.0305) (width 0.2) (layer "F.Cu") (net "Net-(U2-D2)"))
 (segment (start 1194.905 915.895) (end 1196.005 916.995) (width 0.2) (layer "F.Cu") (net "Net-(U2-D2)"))
 (segment (start 1176.616 906.8435) (end 1187.429 896.0305) (width 0.2) (layer "F.Cu") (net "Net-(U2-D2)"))
 (segment (start 1195.360635 929.145) (end 1185.323315 929.145) (width 0.2) (layer "F.Cu") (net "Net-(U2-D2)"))
 (segment (start 1196.005 916.995) (end 1196.005 928.500635) (width 0.2) (layer "F.Cu") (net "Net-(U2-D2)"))
 (segment (start 1143.254 887.984) (end 1143.254 890.037402) (width 0.2) (layer "F.Cu") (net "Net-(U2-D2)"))
 (segment (start 1196.005 928.500635) (end 1195.360635 929.145) (width 0.2) (layer "F.Cu") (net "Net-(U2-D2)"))
 (segment (start 1149.247098 896.0305) (end 1187.429 896.0305) (width 0.2) (layer "F.Cu") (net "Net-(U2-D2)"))
 (segment (start 1158.930101 915.032) (end 1158.11 915.852101) (width 0.2) (layer "B.Cu") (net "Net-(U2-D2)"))
 (segment (start 1158.11 915.852101) (end 1158.11 917.085402) (width 0.2) (layer "B.Cu") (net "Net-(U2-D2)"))
 (segment (start 1159.51 918.485402) (end 1159.51 935.228) (width 0.2) (layer "B.Cu") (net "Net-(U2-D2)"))
 (segment (start 1158.11 917.085402) (end 1159.51 918.485402) (width 0.2) (layer "B.Cu") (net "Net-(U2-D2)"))
 (segment (start 1194.905 915.895) (end 1160.952899 915.895) (width 0.2) (layer "B.Cu") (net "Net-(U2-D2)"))
 (segment (start 1160.089899 915.032) (end 1158.930101 915.032) (width 0.2) (layer "B.Cu") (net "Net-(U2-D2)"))
 (segment (start 1160.952899 915.895) (end 1160.089899 915.032) (width 0.2) (layer "B.Cu") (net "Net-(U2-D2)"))
 (segment (start 1201.519 916.399) (end 1205.065 919.945) (width 0.2) (layer "F.Cu") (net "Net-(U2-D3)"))
 (segment (start 1224.534 887.476) (end 1221.086 884.028) (width 0.2) (layer "F.Cu") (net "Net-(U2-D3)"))
 (segment (start 1189.228 904.108) (end 1189.228 900.3695) (width 0.2) (layer "F.Cu") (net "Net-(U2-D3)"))
 (segment (start 1189.228 900.3695) (end 1187.429 898.5705) (width 0.2) (layer "F.Cu") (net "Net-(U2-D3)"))
 (segment (start 1205.065 919.945) (end 1189.228 904.108) (width 0.2) (layer "F.Cu") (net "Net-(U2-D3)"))
 (segment (start 1189.104 896.8955) (end 1187.429 898.5705) (width 0.2) (layer "F.Cu") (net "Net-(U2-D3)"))
 (segment (start 1197.457186 884.028) (end 1189.104 892.381186) (width 0.2) (layer "F.Cu") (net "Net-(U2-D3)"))
 (segment (start 1189.104 892.381186) (end 1189.104 896.8955) (width 0.2) (layer "F.Cu") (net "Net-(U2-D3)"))
 (segment (start 1221.086 884.028) (end 1197.457186 884.028) (width 0.2) (layer "F.Cu") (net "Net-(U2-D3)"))
 (via (at 1205.065 919.945) (size 0.6) (drill 0.3) (layers "F.Cu" "B.Cu") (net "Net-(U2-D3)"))
 (segment (start 1187.429 906.1905) (end 1187.429 909.859) (width 0.2) (layer "F.Cu") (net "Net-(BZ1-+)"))
 (segment (start 1187.429 909.859) (end 1178.316 918.972) (width 0.2) (layer "F.Cu") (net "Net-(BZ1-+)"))
 (segment (start 1207.991346 902.345) (end 1209.305 901.031346) (width 0.2) (layer "F.Cu") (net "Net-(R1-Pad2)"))
 (segment (start 1231.321585 882.828) (end 1232.684 884.190416) (width 0.2) (layer "F.Cu") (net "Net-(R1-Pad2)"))
 (segment (start 1217.038402 904.645) (end 1207.278654 904.645) (width 0.2) (layer "F.Cu") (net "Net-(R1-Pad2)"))
 (segment (start 1188.796 882.828) (end 1231.321585 882.828) (width 0.2) (layer "F.Cu") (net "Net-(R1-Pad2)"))
 (segment (start 1209.305 893.258654) (end 1208.231346 892.185) (width 0.2) (layer "F.Cu") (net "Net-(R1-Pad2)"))
 (segment (start 1208.231346 892.185) (end 1204.8995 892.185) (width 0.2) (layer "F.Cu") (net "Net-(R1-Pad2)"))
 (segment (start 1206.605 903.018654) (end 1207.278654 902.345) (width 0.2) (layer "F.Cu") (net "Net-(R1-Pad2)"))
 (segment (start 1207.278654 904.645) (end 1206.605 903.971346) (width 0.2) (layer "F.Cu") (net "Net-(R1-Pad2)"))
 (segment (start 1232.684 884.190416) (end 1232.684 888.999402) (width 0.2) (layer "F.Cu") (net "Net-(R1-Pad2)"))
 (segment (start 1232.684 888.999402) (end 1217.038402 904.645) (width 0.2) (layer "F.Cu") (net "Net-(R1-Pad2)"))
 (segment (start 1182.116 889.508) (end 1188.796 882.828) (width 0.2) (layer "F.Cu") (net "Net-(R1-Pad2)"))
 (segment (start 1204.8995 892.185) (end 1203.594 893.4905) (width 0.2) (layer "F.Cu") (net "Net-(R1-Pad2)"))
 (segment (start 1209.305 901.031346) (end 1209.305 893.258654) (width 0.2) (layer "F.Cu") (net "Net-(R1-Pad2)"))
 (segment (start 1207.278654 902.345) (end 1207.991346 902.345) (width 0.2) (layer "F.Cu") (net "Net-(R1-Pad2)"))
 (segment (start 1206.605 903.971346) (end 1206.605 903.018654) (width 0.2) (layer "F.Cu") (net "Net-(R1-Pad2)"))
 (segment (start 1182.116 889.508) (end 1184.519 887.105) (width 0.2) (layer "B.Cu") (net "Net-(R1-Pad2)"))
 (segment (start 1184.519 887.105) (end 1208.903 887.105) (width 0.2) (layer "B.Cu") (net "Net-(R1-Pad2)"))
 (segment (start 1208.905 912.055) (end 1205.065 915.895) (width 0.2) (layer "B.Cu") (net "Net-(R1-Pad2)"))
 (segment (start 1208.903 887.105) (end 1208.905 887.107) (width 0.2) (layer "B.Cu") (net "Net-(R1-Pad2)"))
 (segment (start 1208.905 887.107) (end 1208.905 912.055) (width 0.2) (layer "B.Cu") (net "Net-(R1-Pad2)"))
 (segment (start 1196.754 889.9385) (end 1196.754 890.11) (width 0.2) (layer "F.Cu") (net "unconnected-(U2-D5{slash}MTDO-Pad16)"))
 (segment (start 1196.754 890.11) (end 1196.34 890.524) (width 0.2) (layer "F.Cu") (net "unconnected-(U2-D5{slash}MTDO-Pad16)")))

